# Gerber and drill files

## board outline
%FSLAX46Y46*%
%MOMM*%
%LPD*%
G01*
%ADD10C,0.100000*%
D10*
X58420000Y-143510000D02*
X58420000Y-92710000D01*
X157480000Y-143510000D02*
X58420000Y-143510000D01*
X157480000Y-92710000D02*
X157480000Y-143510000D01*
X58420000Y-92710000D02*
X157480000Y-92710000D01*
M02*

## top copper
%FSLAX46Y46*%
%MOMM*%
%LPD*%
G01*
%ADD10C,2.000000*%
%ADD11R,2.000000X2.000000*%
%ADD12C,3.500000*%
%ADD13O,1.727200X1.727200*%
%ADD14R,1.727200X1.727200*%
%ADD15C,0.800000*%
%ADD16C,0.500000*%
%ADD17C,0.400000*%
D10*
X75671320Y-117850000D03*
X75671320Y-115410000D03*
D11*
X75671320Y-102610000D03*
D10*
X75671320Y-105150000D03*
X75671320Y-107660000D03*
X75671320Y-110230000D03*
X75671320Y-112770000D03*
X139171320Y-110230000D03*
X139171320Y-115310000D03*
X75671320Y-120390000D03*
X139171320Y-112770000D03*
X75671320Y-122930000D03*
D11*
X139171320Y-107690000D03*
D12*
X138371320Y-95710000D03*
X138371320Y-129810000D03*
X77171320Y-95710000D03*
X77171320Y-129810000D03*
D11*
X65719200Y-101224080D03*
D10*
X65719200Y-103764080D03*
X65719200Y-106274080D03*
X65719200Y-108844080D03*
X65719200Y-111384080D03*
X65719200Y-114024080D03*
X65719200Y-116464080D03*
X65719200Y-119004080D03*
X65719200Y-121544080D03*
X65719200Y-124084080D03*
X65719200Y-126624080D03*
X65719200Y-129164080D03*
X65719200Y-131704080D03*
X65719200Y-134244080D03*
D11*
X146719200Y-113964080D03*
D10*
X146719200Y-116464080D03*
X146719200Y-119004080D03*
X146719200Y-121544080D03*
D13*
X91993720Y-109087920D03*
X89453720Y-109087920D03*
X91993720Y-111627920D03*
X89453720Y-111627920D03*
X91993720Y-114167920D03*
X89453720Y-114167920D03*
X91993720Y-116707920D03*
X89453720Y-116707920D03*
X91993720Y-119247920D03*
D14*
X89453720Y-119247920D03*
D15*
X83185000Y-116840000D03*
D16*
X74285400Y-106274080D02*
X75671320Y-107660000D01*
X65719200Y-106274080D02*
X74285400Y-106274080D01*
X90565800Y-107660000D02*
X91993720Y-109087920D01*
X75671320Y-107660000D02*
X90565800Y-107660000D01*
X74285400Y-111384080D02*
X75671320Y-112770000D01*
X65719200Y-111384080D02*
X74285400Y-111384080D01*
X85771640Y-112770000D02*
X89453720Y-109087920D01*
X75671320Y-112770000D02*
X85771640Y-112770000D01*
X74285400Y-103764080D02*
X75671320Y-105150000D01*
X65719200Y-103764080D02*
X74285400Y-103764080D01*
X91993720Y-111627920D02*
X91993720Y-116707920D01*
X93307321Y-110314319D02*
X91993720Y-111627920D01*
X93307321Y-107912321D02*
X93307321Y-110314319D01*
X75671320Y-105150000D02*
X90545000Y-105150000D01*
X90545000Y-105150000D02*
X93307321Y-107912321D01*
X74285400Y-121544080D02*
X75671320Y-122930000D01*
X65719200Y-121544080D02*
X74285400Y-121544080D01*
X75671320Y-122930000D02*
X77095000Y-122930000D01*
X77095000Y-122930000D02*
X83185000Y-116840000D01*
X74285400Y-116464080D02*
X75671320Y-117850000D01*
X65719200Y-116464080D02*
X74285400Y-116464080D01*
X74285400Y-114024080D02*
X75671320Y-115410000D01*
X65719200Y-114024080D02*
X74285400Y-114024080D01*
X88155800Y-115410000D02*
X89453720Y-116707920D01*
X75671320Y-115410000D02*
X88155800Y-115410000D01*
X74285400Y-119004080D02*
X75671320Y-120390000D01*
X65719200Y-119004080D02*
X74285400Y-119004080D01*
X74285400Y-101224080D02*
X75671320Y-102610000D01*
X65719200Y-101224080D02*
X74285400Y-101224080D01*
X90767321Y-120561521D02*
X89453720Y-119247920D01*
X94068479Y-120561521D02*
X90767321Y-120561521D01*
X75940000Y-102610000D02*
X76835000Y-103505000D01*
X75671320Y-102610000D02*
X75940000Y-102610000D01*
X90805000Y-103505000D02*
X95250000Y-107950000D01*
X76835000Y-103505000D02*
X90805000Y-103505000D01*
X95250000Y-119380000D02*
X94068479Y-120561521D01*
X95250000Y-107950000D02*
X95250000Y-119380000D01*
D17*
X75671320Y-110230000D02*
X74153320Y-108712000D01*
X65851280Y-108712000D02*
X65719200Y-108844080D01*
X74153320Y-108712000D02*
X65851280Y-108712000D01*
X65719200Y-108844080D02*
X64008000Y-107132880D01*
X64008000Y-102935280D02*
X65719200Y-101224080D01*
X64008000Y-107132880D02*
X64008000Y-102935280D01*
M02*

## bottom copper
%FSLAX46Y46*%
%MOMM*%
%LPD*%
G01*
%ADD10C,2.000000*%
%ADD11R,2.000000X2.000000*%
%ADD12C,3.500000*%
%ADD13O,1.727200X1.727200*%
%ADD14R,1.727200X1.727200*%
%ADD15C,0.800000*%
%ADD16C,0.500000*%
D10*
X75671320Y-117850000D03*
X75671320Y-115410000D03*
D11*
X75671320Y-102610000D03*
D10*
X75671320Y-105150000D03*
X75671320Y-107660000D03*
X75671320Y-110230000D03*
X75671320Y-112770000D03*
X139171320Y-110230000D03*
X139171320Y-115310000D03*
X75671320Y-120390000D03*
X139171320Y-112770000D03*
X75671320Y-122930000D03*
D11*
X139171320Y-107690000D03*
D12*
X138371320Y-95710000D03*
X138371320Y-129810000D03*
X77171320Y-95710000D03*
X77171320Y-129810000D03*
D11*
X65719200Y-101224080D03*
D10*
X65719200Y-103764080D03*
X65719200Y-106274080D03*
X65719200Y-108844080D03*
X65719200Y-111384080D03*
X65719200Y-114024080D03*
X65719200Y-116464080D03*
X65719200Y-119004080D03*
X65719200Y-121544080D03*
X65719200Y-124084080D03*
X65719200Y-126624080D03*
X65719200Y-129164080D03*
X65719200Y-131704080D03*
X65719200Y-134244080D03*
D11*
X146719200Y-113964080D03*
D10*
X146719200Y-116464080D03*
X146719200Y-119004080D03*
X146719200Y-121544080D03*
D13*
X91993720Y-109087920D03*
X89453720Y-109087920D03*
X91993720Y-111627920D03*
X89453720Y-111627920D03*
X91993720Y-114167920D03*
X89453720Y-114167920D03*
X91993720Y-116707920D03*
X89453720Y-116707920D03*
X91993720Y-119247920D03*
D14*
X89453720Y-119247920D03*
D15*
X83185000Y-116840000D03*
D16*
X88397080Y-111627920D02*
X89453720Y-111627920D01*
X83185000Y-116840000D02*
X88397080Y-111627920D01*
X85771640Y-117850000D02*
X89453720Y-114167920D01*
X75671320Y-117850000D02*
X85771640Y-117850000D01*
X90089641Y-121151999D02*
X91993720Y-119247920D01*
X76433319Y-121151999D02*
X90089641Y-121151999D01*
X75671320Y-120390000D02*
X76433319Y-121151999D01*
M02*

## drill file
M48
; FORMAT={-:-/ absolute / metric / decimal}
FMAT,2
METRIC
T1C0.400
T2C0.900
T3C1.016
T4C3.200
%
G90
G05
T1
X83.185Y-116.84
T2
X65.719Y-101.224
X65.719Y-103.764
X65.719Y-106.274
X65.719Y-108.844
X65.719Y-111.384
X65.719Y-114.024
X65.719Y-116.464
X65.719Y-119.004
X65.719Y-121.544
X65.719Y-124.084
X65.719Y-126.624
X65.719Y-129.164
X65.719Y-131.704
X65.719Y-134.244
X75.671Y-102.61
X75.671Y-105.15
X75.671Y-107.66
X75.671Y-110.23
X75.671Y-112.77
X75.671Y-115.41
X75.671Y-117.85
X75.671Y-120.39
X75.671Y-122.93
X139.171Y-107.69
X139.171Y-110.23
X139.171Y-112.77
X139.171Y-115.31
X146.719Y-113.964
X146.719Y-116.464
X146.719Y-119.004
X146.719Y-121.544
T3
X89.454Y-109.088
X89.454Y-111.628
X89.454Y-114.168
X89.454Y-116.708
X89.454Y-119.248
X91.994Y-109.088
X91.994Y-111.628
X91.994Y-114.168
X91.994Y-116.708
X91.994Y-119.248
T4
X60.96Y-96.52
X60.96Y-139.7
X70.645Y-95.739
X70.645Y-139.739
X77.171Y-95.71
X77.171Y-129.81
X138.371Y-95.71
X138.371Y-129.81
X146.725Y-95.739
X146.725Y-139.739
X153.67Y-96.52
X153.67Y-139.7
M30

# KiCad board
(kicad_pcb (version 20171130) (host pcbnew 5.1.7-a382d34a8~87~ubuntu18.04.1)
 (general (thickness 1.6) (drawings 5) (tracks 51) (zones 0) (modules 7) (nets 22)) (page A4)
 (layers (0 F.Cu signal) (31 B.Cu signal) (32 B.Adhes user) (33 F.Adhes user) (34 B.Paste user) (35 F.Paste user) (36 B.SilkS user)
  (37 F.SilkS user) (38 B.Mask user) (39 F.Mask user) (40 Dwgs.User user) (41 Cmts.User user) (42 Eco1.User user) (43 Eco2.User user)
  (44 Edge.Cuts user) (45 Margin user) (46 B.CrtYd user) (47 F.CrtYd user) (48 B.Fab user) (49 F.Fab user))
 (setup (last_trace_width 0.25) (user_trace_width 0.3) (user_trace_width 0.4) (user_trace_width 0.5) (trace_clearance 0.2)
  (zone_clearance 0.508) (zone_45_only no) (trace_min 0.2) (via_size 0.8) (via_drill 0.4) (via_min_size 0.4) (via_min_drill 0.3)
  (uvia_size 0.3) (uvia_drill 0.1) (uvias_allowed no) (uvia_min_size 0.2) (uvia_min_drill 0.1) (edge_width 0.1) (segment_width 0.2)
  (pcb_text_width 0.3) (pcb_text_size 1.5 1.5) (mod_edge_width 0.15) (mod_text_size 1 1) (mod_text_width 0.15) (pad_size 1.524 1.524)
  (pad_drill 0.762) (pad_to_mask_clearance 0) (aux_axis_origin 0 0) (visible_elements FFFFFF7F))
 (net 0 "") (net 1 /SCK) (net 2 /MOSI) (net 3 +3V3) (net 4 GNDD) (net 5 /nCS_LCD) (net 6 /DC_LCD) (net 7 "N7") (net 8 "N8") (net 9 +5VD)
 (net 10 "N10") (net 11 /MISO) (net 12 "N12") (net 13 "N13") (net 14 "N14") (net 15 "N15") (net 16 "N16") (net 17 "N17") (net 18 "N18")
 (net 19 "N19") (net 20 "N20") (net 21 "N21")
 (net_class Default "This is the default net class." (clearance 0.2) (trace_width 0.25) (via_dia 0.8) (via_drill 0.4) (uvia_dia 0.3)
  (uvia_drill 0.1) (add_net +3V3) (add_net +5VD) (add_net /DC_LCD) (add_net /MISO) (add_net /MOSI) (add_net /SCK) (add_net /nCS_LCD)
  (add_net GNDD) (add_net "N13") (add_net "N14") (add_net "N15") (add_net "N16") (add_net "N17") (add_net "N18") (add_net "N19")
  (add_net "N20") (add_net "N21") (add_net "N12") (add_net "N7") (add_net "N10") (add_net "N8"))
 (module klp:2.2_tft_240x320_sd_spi (layer F.Cu) (at 109.77372 112.776 270)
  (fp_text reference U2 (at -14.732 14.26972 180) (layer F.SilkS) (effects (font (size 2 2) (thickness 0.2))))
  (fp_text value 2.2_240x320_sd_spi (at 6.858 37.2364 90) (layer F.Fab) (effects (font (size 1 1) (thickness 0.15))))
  (pad 7 thru_hole circle (at 5.074 34.1024 270) (size 2 2) (drill 0.9) (layers *.Cu *.Mask) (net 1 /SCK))
  (pad 6 thru_hole circle (at 2.634 34.1024 270) (size 2 2) (drill 0.9) (layers *.Cu *.Mask) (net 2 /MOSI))
  (pad 1 thru_hole rect (at -10.166 34.1024 270) (size 2 2) (drill 0.9) (layers *.Cu *.Mask) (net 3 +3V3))
  (pad 2 thru_hole circle (at -7.626 34.1024 270) (size 2 2) (drill 0.9) (layers *.Cu *.Mask) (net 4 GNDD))
  (pad 3 thru_hole circle (at -5.116 34.1024 270) (size 2 2) (drill 0.9) (layers *.Cu *.Mask) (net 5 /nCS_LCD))
  (pad 4 thru_hole circle (at -2.546 34.1024 270) (size 2 2) (drill 0.9) (layers *.Cu *.Mask) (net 3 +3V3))
  (pad 5 thru_hole circle (at -0.006 34.1024 270) (size 2 2) (drill 0.9) (layers *.Cu *.Mask) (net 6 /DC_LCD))
  (pad 16 thru_hole circle (at -2.546 -29.3976 270) (size 2 2) (drill 0.9) (layers *.Cu *.Mask) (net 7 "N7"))
  (pad 18 thru_hole circle (at 2.534 -29.3976 270) (size 2 2) (drill 0.9) (layers *.Cu *.Mask) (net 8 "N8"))
  (pad 8 thru_hole circle (at 7.614 34.1024 270) (size 2 2) (drill 0.9) (layers *.Cu *.Mask) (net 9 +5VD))
  (pad 17 thru_hole circle (at -0.006 -29.3976 270) (size 2 2) (drill 0.9) (layers *.Cu *.Mask) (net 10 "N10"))
  (pad 9 thru_hole circle (at 10.154 34.1024 270) (size 2 2) (drill 0.9) (layers *.Cu *.Mask) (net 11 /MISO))
  (pad 15 thru_hole rect (at -5.086 -29.3976 270) (size 2 2) (drill 0.9) (layers *.Cu *.Mask) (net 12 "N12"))
  (pad "" np_thru_hole circle (at -17.066 -28.5976 270) (size 3.5 3.5) (drill 3.2) (layers *.Cu *.Mask))
  (pad "" np_thru_hole circle (at 17.034 -28.5976 270) (size 3.5 3.5) (drill 3.2) (layers *.Cu *.Mask))
  (pad "" np_thru_hole circle (at -17.066 32.6024 270) (size 3.5 3.5) (drill 3.2) (layers *.Cu *.Mask))
  (pad "" np_thru_hole circle (at 17.034 32.6024 270) (size 3.5 3.5) (drill 3.2) (layers *.Cu *.Mask)))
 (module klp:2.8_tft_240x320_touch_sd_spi (layer F.Cu) (at 112.07496 117.73916 270)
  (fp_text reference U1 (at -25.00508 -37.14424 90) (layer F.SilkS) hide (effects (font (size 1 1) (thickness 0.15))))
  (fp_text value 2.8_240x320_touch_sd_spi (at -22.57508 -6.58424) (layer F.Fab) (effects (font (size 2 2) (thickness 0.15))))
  (pad 1 thru_hole rect (at -16.51508 46.35576 270) (size 2 2) (drill 0.9) (layers *.Cu *.Mask) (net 3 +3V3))
  (pad 2 thru_hole circle (at -13.97508 46.35576 270) (size 2 2) (drill 0.9) (layers *.Cu *.Mask) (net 4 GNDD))
  (pad 3 thru_hole circle (at -11.46508 46.35576 270) (size 2 2) (drill 0.9) (layers *.Cu *.Mask) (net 5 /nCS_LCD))
  (pad 4 thru_hole circle (at -8.89508 46.35576 270) (size 2 2) (drill 0.9) (layers *.Cu *.Mask) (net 3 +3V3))
  (pad 5 thru_hole circle (at -6.35508 46.35576 270) (size 2 2) (drill 0.9) (layers *.Cu *.Mask) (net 6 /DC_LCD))
  (pad 6 thru_hole circle (at -3.71508 46.35576 270) (size 2 2) (drill 0.9) (layers *.Cu *.Mask) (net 2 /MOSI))
  (pad 7 thru_hole circle (at -1.27508 46.35576 270) (size 2 2) (drill 0.9) (layers *.Cu *.Mask) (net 1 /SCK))
  (pad 8 thru_hole circle (at 1.26492 46.35576 270) (size 2 2) (drill 0.9) (layers *.Cu *.Mask) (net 9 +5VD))
  (pad 9 thru_hole circle (at 3.80492 46.35576 270) (size 2 2) (drill 0.9) (layers *.Cu *.Mask) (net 11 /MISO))
  (pad 10 thru_hole circle (at 6.34492 46.35576 270) (size 2 2) (drill 0.9) (layers *.Cu *.Mask) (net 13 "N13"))
  (pad 11 thru_hole circle (at 8.88492 46.35576 270) (size 2 2) (drill 0.9) (layers *.Cu *.Mask) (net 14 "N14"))
  (pad 12 thru_hole circle (at 11.42492 46.35576 270) (size 2 2) (drill 0.9) (layers *.Cu *.Mask) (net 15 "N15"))
  (pad 13 thru_hole circle (at 13.96492 46.35576 270) (size 2 2) (drill 0.9) (layers *.Cu *.Mask) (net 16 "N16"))
  (pad 14 thru_hole circle (at 16.50492 46.35576 270) (size 2 2) (drill 0.9) (layers *.Cu *.Mask) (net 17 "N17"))
  (pad 15 thru_hole rect (at -3.77508 -34.64424 270) (size 2 2) (drill 0.9) (layers *.Cu *.Mask) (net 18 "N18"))
  (pad 16 thru_hole circle (at -1.27508 -34.64424 270) (size 2 2) (drill 0.9) (layers *.Cu *.Mask) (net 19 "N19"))
  (pad 17 thru_hole circle (at 1.26492 -34.64424 270) (size 2 2) (drill 0.9) (layers *.Cu *.Mask) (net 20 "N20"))
  (pad 18 thru_hole circle (at 3.80492 -34.64424 270) (size 2 2) (drill 0.9) (layers *.Cu *.Mask) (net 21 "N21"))
  (pad "" np_thru_hole circle (at -22 41.43 270) (size 3.2 3.2) (drill 3.2) (layers *.Cu *.Mask))
  (pad "" np_thru_hole circle (at 22 41.43 270) (size 3.2 3.2) (drill 3.2) (layers *.Cu *.Mask))
  (pad "" np_thru_hole circle (at -22 -34.65 270) (size 3.2 3.2) (drill 3.2) (layers *.Cu *.Mask))
  (pad "" np_thru_hole circle (at 22 -34.65 270) (size 3.2 3.2) (drill 3.2) (layers *.Cu *.Mask)))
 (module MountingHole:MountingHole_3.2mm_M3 (layer F.Cu) (at 153.67 139.7)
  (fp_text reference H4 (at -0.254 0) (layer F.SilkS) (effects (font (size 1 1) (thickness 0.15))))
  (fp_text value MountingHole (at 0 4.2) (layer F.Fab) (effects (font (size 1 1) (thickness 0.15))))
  (pad 1 np_thru_hole circle (at 0 0) (size 3.2 3.2) (drill 3.2) (layers *.Cu *.Mask)))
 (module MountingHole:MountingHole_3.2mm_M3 (layer F.Cu) (at 60.96 139.7)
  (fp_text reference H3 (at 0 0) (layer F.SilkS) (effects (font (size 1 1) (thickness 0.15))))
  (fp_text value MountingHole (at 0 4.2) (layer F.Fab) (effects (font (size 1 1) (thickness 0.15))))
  (pad 1 np_thru_hole circle (at 0 0) (size 3.2 3.2) (drill 3.2) (layers *.Cu *.Mask)))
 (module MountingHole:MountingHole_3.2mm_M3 (layer F.Cu) (at 153.67 96.52)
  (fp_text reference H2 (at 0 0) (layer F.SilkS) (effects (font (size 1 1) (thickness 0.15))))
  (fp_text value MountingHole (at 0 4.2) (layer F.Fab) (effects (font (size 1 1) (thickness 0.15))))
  (pad 1 np_thru_hole circle (at 0 0) (size 3.2 3.2) (drill 3.2) (layers *.Cu *.Mask)))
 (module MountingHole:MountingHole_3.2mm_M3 (layer F.Cu) (at 60.96 96.52)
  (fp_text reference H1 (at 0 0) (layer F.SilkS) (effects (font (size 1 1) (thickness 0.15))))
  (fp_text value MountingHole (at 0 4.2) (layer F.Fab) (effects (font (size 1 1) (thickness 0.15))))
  (pad 1 np_thru_hole circle (at 0 0) (size 3.2 3.2) (drill 3.2) (layers *.Cu *.Mask)))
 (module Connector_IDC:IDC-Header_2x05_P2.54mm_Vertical (layer B.Cu) (at 89.45372 119.24792)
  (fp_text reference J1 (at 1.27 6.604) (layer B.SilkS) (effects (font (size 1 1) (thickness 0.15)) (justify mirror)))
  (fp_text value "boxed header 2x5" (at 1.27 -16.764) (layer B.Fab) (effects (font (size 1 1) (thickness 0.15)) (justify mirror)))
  (pad 10 thru_hole oval (at 2.54 -10.16) (size 1.7272 1.7272) (drill 1.016) (layers *.Cu *.Mask) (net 5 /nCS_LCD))
  (pad 9 thru_hole oval (at 0 -10.16) (size 1.7272 1.7272) (drill 1.016) (layers *.Cu *.Mask) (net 6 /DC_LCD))
  (pad 8 thru_hole oval (at 2.54 -7.62) (size 1.7272 1.7272) (drill 1.016) (layers *.Cu *.Mask) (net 4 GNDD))
  (pad 7 thru_hole oval (at 0 -7.62) (size 1.7272 1.7272) (drill 1.016) (layers *.Cu *.Mask) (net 11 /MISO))
  (pad 6 thru_hole oval (at 2.54 -5.08) (size 1.7272 1.7272) (drill 1.016) (layers *.Cu *.Mask) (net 4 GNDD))
  (pad 5 thru_hole oval (at 0 -5.08) (size 1.7272 1.7272) (drill 1.016) (layers *.Cu *.Mask) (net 1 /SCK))
  (pad 4 thru_hole oval (at 2.54 -2.54) (size 1.7272 1.7272) (drill 1.016) (layers *.Cu *.Mask) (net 4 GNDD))
  (pad 3 thru_hole oval (at 0 -2.54) (size 1.7272 1.7272) (drill 1.016) (layers *.Cu *.Mask) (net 2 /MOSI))
  (pad 2 thru_hole oval (at 2.54 0) (size 1.7272 1.7272) (drill 1.016) (layers *.Cu *.Mask) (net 9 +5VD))
  (pad 1 thru_hole rect (at 0 0) (size 1.7272 1.7272) (drill 1.016) (layers *.Cu *.Mask) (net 3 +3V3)))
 (gr_line (start 58.42 143.51) (end 58.42 92.71) (layer Edge.Cuts) (width 0.1))
 (gr_line (start 157.48 143.51) (end 58.42 143.51) (layer Edge.Cuts) (width 0.1))
 (gr_line (start 157.48 92.71) (end 157.48 143.51) (layer Edge.Cuts) (width 0.1))
 (gr_line (start 58.42 92.71) (end 157.48 92.71) (layer Edge.Cuts) (width 0.1))
 (segment (start 74.2854 106.27408) (end 75.67132 107.66) (width 0.5) (layer F.Cu) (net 5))
 (segment (start 65.7192 106.27408) (end 74.2854 106.27408) (width 0.5) (layer F.Cu) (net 5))
 (segment (start 90.5658 107.66) (end 91.99372 109.08792) (width 0.5) (layer F.Cu) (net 5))
 (segment (start 75.67132 107.66) (end 90.5658 107.66) (width 0.5) (layer F.Cu) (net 5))
 (segment (start 74.2854 111.38408) (end 75.67132 112.77) (width 0.5) (layer F.Cu) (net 6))
 (segment (start 65.7192 111.38408) (end 74.2854 111.38408) (width 0.5) (layer F.Cu) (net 6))
 (segment (start 85.77164 112.77) (end 89.45372 109.08792) (width 0.5) (layer F.Cu) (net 6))
 (segment (start 75.67132 112.77) (end 85.77164 112.77) (width 0.5) (layer F.Cu) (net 6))
 (segment (start 74.2854 103.76408) (end 75.67132 105.15) (width 0.5) (layer F.Cu) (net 4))
 (segment (start 65.7192 103.76408) (end 74.2854 103.76408) (width 0.5) (layer F.Cu) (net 4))
 (segment (start 91.99372 111.62792) (end 91.99372 116.70792) (width 0.5) (layer F.Cu) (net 4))
 (segment (start 93.307321 110.314319) (end 91.99372 111.62792) (width 0.5) (layer F.Cu) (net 4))
 (segment (start 93.307321 107.912321) (end 93.307321 110.314319) (width 0.5) (layer F.Cu) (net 4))
 (segment (start 75.67132 105.15) (end 90.545 105.15) (width 0.5) (layer F.Cu) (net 4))
 (segment (start 90.545 105.15) (end 93.307321 107.912321) (width 0.5) (layer F.Cu) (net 4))
 (segment (start 74.2854 121.54408) (end 75.67132 122.93) (width 0.5) (layer F.Cu) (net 11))
 (segment (start 65.7192 121.54408) (end 74.2854 121.54408) (width 0.5) (layer F.Cu) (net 11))
 (via (at 83.185 116.84) (size 0.8) (drill 0.4) (layers F.Cu B.Cu) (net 11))
 (segment (start 75.67132 122.93) (end 77.095 122.93) (width 0.5) (layer F.Cu) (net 11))
 (segment (start 77.095 122.93) (end 83.185 116.84) (width 0.5) (layer F.Cu) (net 11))
 (segment (start 88.39708 111.62792) (end 89.45372 111.62792) (width 0.5) (layer B.Cu) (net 11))
 (segment (start 83.185 116.84) (end 88.39708 111.62792) (width 0.5) (layer B.Cu) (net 11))
 (segment (start 74.2854 116.46408) (end 75.67132 117.85) (width 0.5) (layer F.Cu) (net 1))
 (segment (start 65.7192 116.46408) (end 74.2854 116.46408) (width 0.5) (layer F.Cu) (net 1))
 (segment (start 85.77164 117.85) (end 89.45372 114.16792) (width 0.5) (layer B.Cu) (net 1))
 (segment (start 75.67132 117.85) (end 85.77164 117.85) (width 0.5) (layer B.Cu) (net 1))
 (segment (start 74.2854 114.02408) (end 75.67132 115.41) (width 0.5) (layer F.Cu) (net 2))
 (segment (start 65.7192 114.02408) (end 74.2854 114.02408) (width 0.5) (layer F.Cu) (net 2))
 (segment (start 88.1558 115.41) (end 89.45372 116.70792) (width 0.5) (layer F.Cu) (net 2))
 (segment (start 75.67132 115.41) (end 88.1558 115.41) (width 0.5) (layer F.Cu) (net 2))
 (segment (start 74.2854 119.00408) (end 75.67132 120.39) (width 0.5) (layer F.Cu) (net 9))
 (segment (start 65.7192 119.00408) (end 74.2854 119.00408) (width 0.5) (layer F.Cu) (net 9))
 (segment (start 90.089641 121.151999) (end 91.99372 119.24792) (width 0.5) (layer B.Cu) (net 9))
 (segment (start 76.433319 121.151999) (end 90.089641 121.151999) (width 0.5) (layer B.Cu) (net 9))
 (segment (start 75.67132 120.39) (end 76.433319 121.151999) (width 0.5) (layer B.Cu) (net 9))
 (segment (start 74.2854 101.22408) (end 75.67132 102.61) (width 0.5) (layer F.Cu) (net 3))
 (segment (start 65.7192 101.22408) (end 74.2854 101.22408) (width 0.5) (layer F.Cu) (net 3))
 (segment (start 90.767321 120.561521) (end 89.45372 119.24792) (width 0.5) (layer F.Cu) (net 3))
 (segment (start 94.068479 120.561521) (end 90.767321 120.561521) (width 0.5) (layer F.Cu) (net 3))
 (segment (start 75.94 102.61) (end 76.835 103.505) (width 0.5) (layer F.Cu) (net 3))
 (segment (start 75.67132 102.61) (end 75.94 102.61) (width 0.5) (layer F.Cu) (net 3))
 (segment (start 90.805 103.505) (end 95.25 107.95) (width 0.5) (layer F.Cu) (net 3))
 (segment (start 76.835 103.505) (end 90.805 103.505) (width 0.5) (layer F.Cu) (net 3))
 (segment (start 95.25 119.38) (end 94.068479 120.561521) (width 0.5) (layer F.Cu) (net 3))
 (segment (start 95.25 107.95) (end 95.25 119.38) (width 0.5) (layer F.Cu) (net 3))
 (segment (start 75.67132 110.23) (end 74.15332 108.712) (width 0.4) (layer F.Cu) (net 3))
 (segment (start 65.85128 108.712) (end 65.7192 108.84408) (width 0.4) (layer F.Cu) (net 3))
 (segment (start 74.15332 108.712) (end 65.85128 108.712) (width 0.4) (layer F.Cu) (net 3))
 (segment (start 65.7192 108.84408) (end 64.008 107.13288) (width 0.4) (layer F.Cu) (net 3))
 (segment (start 64.008 102.93528) (end 65.7192 101.22408) (width 0.4) (layer F.Cu) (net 3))
 (segment (start 64.008 107.13288) (end 64.008 102.93528) (width 0.4) (layer F.Cu) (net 3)))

